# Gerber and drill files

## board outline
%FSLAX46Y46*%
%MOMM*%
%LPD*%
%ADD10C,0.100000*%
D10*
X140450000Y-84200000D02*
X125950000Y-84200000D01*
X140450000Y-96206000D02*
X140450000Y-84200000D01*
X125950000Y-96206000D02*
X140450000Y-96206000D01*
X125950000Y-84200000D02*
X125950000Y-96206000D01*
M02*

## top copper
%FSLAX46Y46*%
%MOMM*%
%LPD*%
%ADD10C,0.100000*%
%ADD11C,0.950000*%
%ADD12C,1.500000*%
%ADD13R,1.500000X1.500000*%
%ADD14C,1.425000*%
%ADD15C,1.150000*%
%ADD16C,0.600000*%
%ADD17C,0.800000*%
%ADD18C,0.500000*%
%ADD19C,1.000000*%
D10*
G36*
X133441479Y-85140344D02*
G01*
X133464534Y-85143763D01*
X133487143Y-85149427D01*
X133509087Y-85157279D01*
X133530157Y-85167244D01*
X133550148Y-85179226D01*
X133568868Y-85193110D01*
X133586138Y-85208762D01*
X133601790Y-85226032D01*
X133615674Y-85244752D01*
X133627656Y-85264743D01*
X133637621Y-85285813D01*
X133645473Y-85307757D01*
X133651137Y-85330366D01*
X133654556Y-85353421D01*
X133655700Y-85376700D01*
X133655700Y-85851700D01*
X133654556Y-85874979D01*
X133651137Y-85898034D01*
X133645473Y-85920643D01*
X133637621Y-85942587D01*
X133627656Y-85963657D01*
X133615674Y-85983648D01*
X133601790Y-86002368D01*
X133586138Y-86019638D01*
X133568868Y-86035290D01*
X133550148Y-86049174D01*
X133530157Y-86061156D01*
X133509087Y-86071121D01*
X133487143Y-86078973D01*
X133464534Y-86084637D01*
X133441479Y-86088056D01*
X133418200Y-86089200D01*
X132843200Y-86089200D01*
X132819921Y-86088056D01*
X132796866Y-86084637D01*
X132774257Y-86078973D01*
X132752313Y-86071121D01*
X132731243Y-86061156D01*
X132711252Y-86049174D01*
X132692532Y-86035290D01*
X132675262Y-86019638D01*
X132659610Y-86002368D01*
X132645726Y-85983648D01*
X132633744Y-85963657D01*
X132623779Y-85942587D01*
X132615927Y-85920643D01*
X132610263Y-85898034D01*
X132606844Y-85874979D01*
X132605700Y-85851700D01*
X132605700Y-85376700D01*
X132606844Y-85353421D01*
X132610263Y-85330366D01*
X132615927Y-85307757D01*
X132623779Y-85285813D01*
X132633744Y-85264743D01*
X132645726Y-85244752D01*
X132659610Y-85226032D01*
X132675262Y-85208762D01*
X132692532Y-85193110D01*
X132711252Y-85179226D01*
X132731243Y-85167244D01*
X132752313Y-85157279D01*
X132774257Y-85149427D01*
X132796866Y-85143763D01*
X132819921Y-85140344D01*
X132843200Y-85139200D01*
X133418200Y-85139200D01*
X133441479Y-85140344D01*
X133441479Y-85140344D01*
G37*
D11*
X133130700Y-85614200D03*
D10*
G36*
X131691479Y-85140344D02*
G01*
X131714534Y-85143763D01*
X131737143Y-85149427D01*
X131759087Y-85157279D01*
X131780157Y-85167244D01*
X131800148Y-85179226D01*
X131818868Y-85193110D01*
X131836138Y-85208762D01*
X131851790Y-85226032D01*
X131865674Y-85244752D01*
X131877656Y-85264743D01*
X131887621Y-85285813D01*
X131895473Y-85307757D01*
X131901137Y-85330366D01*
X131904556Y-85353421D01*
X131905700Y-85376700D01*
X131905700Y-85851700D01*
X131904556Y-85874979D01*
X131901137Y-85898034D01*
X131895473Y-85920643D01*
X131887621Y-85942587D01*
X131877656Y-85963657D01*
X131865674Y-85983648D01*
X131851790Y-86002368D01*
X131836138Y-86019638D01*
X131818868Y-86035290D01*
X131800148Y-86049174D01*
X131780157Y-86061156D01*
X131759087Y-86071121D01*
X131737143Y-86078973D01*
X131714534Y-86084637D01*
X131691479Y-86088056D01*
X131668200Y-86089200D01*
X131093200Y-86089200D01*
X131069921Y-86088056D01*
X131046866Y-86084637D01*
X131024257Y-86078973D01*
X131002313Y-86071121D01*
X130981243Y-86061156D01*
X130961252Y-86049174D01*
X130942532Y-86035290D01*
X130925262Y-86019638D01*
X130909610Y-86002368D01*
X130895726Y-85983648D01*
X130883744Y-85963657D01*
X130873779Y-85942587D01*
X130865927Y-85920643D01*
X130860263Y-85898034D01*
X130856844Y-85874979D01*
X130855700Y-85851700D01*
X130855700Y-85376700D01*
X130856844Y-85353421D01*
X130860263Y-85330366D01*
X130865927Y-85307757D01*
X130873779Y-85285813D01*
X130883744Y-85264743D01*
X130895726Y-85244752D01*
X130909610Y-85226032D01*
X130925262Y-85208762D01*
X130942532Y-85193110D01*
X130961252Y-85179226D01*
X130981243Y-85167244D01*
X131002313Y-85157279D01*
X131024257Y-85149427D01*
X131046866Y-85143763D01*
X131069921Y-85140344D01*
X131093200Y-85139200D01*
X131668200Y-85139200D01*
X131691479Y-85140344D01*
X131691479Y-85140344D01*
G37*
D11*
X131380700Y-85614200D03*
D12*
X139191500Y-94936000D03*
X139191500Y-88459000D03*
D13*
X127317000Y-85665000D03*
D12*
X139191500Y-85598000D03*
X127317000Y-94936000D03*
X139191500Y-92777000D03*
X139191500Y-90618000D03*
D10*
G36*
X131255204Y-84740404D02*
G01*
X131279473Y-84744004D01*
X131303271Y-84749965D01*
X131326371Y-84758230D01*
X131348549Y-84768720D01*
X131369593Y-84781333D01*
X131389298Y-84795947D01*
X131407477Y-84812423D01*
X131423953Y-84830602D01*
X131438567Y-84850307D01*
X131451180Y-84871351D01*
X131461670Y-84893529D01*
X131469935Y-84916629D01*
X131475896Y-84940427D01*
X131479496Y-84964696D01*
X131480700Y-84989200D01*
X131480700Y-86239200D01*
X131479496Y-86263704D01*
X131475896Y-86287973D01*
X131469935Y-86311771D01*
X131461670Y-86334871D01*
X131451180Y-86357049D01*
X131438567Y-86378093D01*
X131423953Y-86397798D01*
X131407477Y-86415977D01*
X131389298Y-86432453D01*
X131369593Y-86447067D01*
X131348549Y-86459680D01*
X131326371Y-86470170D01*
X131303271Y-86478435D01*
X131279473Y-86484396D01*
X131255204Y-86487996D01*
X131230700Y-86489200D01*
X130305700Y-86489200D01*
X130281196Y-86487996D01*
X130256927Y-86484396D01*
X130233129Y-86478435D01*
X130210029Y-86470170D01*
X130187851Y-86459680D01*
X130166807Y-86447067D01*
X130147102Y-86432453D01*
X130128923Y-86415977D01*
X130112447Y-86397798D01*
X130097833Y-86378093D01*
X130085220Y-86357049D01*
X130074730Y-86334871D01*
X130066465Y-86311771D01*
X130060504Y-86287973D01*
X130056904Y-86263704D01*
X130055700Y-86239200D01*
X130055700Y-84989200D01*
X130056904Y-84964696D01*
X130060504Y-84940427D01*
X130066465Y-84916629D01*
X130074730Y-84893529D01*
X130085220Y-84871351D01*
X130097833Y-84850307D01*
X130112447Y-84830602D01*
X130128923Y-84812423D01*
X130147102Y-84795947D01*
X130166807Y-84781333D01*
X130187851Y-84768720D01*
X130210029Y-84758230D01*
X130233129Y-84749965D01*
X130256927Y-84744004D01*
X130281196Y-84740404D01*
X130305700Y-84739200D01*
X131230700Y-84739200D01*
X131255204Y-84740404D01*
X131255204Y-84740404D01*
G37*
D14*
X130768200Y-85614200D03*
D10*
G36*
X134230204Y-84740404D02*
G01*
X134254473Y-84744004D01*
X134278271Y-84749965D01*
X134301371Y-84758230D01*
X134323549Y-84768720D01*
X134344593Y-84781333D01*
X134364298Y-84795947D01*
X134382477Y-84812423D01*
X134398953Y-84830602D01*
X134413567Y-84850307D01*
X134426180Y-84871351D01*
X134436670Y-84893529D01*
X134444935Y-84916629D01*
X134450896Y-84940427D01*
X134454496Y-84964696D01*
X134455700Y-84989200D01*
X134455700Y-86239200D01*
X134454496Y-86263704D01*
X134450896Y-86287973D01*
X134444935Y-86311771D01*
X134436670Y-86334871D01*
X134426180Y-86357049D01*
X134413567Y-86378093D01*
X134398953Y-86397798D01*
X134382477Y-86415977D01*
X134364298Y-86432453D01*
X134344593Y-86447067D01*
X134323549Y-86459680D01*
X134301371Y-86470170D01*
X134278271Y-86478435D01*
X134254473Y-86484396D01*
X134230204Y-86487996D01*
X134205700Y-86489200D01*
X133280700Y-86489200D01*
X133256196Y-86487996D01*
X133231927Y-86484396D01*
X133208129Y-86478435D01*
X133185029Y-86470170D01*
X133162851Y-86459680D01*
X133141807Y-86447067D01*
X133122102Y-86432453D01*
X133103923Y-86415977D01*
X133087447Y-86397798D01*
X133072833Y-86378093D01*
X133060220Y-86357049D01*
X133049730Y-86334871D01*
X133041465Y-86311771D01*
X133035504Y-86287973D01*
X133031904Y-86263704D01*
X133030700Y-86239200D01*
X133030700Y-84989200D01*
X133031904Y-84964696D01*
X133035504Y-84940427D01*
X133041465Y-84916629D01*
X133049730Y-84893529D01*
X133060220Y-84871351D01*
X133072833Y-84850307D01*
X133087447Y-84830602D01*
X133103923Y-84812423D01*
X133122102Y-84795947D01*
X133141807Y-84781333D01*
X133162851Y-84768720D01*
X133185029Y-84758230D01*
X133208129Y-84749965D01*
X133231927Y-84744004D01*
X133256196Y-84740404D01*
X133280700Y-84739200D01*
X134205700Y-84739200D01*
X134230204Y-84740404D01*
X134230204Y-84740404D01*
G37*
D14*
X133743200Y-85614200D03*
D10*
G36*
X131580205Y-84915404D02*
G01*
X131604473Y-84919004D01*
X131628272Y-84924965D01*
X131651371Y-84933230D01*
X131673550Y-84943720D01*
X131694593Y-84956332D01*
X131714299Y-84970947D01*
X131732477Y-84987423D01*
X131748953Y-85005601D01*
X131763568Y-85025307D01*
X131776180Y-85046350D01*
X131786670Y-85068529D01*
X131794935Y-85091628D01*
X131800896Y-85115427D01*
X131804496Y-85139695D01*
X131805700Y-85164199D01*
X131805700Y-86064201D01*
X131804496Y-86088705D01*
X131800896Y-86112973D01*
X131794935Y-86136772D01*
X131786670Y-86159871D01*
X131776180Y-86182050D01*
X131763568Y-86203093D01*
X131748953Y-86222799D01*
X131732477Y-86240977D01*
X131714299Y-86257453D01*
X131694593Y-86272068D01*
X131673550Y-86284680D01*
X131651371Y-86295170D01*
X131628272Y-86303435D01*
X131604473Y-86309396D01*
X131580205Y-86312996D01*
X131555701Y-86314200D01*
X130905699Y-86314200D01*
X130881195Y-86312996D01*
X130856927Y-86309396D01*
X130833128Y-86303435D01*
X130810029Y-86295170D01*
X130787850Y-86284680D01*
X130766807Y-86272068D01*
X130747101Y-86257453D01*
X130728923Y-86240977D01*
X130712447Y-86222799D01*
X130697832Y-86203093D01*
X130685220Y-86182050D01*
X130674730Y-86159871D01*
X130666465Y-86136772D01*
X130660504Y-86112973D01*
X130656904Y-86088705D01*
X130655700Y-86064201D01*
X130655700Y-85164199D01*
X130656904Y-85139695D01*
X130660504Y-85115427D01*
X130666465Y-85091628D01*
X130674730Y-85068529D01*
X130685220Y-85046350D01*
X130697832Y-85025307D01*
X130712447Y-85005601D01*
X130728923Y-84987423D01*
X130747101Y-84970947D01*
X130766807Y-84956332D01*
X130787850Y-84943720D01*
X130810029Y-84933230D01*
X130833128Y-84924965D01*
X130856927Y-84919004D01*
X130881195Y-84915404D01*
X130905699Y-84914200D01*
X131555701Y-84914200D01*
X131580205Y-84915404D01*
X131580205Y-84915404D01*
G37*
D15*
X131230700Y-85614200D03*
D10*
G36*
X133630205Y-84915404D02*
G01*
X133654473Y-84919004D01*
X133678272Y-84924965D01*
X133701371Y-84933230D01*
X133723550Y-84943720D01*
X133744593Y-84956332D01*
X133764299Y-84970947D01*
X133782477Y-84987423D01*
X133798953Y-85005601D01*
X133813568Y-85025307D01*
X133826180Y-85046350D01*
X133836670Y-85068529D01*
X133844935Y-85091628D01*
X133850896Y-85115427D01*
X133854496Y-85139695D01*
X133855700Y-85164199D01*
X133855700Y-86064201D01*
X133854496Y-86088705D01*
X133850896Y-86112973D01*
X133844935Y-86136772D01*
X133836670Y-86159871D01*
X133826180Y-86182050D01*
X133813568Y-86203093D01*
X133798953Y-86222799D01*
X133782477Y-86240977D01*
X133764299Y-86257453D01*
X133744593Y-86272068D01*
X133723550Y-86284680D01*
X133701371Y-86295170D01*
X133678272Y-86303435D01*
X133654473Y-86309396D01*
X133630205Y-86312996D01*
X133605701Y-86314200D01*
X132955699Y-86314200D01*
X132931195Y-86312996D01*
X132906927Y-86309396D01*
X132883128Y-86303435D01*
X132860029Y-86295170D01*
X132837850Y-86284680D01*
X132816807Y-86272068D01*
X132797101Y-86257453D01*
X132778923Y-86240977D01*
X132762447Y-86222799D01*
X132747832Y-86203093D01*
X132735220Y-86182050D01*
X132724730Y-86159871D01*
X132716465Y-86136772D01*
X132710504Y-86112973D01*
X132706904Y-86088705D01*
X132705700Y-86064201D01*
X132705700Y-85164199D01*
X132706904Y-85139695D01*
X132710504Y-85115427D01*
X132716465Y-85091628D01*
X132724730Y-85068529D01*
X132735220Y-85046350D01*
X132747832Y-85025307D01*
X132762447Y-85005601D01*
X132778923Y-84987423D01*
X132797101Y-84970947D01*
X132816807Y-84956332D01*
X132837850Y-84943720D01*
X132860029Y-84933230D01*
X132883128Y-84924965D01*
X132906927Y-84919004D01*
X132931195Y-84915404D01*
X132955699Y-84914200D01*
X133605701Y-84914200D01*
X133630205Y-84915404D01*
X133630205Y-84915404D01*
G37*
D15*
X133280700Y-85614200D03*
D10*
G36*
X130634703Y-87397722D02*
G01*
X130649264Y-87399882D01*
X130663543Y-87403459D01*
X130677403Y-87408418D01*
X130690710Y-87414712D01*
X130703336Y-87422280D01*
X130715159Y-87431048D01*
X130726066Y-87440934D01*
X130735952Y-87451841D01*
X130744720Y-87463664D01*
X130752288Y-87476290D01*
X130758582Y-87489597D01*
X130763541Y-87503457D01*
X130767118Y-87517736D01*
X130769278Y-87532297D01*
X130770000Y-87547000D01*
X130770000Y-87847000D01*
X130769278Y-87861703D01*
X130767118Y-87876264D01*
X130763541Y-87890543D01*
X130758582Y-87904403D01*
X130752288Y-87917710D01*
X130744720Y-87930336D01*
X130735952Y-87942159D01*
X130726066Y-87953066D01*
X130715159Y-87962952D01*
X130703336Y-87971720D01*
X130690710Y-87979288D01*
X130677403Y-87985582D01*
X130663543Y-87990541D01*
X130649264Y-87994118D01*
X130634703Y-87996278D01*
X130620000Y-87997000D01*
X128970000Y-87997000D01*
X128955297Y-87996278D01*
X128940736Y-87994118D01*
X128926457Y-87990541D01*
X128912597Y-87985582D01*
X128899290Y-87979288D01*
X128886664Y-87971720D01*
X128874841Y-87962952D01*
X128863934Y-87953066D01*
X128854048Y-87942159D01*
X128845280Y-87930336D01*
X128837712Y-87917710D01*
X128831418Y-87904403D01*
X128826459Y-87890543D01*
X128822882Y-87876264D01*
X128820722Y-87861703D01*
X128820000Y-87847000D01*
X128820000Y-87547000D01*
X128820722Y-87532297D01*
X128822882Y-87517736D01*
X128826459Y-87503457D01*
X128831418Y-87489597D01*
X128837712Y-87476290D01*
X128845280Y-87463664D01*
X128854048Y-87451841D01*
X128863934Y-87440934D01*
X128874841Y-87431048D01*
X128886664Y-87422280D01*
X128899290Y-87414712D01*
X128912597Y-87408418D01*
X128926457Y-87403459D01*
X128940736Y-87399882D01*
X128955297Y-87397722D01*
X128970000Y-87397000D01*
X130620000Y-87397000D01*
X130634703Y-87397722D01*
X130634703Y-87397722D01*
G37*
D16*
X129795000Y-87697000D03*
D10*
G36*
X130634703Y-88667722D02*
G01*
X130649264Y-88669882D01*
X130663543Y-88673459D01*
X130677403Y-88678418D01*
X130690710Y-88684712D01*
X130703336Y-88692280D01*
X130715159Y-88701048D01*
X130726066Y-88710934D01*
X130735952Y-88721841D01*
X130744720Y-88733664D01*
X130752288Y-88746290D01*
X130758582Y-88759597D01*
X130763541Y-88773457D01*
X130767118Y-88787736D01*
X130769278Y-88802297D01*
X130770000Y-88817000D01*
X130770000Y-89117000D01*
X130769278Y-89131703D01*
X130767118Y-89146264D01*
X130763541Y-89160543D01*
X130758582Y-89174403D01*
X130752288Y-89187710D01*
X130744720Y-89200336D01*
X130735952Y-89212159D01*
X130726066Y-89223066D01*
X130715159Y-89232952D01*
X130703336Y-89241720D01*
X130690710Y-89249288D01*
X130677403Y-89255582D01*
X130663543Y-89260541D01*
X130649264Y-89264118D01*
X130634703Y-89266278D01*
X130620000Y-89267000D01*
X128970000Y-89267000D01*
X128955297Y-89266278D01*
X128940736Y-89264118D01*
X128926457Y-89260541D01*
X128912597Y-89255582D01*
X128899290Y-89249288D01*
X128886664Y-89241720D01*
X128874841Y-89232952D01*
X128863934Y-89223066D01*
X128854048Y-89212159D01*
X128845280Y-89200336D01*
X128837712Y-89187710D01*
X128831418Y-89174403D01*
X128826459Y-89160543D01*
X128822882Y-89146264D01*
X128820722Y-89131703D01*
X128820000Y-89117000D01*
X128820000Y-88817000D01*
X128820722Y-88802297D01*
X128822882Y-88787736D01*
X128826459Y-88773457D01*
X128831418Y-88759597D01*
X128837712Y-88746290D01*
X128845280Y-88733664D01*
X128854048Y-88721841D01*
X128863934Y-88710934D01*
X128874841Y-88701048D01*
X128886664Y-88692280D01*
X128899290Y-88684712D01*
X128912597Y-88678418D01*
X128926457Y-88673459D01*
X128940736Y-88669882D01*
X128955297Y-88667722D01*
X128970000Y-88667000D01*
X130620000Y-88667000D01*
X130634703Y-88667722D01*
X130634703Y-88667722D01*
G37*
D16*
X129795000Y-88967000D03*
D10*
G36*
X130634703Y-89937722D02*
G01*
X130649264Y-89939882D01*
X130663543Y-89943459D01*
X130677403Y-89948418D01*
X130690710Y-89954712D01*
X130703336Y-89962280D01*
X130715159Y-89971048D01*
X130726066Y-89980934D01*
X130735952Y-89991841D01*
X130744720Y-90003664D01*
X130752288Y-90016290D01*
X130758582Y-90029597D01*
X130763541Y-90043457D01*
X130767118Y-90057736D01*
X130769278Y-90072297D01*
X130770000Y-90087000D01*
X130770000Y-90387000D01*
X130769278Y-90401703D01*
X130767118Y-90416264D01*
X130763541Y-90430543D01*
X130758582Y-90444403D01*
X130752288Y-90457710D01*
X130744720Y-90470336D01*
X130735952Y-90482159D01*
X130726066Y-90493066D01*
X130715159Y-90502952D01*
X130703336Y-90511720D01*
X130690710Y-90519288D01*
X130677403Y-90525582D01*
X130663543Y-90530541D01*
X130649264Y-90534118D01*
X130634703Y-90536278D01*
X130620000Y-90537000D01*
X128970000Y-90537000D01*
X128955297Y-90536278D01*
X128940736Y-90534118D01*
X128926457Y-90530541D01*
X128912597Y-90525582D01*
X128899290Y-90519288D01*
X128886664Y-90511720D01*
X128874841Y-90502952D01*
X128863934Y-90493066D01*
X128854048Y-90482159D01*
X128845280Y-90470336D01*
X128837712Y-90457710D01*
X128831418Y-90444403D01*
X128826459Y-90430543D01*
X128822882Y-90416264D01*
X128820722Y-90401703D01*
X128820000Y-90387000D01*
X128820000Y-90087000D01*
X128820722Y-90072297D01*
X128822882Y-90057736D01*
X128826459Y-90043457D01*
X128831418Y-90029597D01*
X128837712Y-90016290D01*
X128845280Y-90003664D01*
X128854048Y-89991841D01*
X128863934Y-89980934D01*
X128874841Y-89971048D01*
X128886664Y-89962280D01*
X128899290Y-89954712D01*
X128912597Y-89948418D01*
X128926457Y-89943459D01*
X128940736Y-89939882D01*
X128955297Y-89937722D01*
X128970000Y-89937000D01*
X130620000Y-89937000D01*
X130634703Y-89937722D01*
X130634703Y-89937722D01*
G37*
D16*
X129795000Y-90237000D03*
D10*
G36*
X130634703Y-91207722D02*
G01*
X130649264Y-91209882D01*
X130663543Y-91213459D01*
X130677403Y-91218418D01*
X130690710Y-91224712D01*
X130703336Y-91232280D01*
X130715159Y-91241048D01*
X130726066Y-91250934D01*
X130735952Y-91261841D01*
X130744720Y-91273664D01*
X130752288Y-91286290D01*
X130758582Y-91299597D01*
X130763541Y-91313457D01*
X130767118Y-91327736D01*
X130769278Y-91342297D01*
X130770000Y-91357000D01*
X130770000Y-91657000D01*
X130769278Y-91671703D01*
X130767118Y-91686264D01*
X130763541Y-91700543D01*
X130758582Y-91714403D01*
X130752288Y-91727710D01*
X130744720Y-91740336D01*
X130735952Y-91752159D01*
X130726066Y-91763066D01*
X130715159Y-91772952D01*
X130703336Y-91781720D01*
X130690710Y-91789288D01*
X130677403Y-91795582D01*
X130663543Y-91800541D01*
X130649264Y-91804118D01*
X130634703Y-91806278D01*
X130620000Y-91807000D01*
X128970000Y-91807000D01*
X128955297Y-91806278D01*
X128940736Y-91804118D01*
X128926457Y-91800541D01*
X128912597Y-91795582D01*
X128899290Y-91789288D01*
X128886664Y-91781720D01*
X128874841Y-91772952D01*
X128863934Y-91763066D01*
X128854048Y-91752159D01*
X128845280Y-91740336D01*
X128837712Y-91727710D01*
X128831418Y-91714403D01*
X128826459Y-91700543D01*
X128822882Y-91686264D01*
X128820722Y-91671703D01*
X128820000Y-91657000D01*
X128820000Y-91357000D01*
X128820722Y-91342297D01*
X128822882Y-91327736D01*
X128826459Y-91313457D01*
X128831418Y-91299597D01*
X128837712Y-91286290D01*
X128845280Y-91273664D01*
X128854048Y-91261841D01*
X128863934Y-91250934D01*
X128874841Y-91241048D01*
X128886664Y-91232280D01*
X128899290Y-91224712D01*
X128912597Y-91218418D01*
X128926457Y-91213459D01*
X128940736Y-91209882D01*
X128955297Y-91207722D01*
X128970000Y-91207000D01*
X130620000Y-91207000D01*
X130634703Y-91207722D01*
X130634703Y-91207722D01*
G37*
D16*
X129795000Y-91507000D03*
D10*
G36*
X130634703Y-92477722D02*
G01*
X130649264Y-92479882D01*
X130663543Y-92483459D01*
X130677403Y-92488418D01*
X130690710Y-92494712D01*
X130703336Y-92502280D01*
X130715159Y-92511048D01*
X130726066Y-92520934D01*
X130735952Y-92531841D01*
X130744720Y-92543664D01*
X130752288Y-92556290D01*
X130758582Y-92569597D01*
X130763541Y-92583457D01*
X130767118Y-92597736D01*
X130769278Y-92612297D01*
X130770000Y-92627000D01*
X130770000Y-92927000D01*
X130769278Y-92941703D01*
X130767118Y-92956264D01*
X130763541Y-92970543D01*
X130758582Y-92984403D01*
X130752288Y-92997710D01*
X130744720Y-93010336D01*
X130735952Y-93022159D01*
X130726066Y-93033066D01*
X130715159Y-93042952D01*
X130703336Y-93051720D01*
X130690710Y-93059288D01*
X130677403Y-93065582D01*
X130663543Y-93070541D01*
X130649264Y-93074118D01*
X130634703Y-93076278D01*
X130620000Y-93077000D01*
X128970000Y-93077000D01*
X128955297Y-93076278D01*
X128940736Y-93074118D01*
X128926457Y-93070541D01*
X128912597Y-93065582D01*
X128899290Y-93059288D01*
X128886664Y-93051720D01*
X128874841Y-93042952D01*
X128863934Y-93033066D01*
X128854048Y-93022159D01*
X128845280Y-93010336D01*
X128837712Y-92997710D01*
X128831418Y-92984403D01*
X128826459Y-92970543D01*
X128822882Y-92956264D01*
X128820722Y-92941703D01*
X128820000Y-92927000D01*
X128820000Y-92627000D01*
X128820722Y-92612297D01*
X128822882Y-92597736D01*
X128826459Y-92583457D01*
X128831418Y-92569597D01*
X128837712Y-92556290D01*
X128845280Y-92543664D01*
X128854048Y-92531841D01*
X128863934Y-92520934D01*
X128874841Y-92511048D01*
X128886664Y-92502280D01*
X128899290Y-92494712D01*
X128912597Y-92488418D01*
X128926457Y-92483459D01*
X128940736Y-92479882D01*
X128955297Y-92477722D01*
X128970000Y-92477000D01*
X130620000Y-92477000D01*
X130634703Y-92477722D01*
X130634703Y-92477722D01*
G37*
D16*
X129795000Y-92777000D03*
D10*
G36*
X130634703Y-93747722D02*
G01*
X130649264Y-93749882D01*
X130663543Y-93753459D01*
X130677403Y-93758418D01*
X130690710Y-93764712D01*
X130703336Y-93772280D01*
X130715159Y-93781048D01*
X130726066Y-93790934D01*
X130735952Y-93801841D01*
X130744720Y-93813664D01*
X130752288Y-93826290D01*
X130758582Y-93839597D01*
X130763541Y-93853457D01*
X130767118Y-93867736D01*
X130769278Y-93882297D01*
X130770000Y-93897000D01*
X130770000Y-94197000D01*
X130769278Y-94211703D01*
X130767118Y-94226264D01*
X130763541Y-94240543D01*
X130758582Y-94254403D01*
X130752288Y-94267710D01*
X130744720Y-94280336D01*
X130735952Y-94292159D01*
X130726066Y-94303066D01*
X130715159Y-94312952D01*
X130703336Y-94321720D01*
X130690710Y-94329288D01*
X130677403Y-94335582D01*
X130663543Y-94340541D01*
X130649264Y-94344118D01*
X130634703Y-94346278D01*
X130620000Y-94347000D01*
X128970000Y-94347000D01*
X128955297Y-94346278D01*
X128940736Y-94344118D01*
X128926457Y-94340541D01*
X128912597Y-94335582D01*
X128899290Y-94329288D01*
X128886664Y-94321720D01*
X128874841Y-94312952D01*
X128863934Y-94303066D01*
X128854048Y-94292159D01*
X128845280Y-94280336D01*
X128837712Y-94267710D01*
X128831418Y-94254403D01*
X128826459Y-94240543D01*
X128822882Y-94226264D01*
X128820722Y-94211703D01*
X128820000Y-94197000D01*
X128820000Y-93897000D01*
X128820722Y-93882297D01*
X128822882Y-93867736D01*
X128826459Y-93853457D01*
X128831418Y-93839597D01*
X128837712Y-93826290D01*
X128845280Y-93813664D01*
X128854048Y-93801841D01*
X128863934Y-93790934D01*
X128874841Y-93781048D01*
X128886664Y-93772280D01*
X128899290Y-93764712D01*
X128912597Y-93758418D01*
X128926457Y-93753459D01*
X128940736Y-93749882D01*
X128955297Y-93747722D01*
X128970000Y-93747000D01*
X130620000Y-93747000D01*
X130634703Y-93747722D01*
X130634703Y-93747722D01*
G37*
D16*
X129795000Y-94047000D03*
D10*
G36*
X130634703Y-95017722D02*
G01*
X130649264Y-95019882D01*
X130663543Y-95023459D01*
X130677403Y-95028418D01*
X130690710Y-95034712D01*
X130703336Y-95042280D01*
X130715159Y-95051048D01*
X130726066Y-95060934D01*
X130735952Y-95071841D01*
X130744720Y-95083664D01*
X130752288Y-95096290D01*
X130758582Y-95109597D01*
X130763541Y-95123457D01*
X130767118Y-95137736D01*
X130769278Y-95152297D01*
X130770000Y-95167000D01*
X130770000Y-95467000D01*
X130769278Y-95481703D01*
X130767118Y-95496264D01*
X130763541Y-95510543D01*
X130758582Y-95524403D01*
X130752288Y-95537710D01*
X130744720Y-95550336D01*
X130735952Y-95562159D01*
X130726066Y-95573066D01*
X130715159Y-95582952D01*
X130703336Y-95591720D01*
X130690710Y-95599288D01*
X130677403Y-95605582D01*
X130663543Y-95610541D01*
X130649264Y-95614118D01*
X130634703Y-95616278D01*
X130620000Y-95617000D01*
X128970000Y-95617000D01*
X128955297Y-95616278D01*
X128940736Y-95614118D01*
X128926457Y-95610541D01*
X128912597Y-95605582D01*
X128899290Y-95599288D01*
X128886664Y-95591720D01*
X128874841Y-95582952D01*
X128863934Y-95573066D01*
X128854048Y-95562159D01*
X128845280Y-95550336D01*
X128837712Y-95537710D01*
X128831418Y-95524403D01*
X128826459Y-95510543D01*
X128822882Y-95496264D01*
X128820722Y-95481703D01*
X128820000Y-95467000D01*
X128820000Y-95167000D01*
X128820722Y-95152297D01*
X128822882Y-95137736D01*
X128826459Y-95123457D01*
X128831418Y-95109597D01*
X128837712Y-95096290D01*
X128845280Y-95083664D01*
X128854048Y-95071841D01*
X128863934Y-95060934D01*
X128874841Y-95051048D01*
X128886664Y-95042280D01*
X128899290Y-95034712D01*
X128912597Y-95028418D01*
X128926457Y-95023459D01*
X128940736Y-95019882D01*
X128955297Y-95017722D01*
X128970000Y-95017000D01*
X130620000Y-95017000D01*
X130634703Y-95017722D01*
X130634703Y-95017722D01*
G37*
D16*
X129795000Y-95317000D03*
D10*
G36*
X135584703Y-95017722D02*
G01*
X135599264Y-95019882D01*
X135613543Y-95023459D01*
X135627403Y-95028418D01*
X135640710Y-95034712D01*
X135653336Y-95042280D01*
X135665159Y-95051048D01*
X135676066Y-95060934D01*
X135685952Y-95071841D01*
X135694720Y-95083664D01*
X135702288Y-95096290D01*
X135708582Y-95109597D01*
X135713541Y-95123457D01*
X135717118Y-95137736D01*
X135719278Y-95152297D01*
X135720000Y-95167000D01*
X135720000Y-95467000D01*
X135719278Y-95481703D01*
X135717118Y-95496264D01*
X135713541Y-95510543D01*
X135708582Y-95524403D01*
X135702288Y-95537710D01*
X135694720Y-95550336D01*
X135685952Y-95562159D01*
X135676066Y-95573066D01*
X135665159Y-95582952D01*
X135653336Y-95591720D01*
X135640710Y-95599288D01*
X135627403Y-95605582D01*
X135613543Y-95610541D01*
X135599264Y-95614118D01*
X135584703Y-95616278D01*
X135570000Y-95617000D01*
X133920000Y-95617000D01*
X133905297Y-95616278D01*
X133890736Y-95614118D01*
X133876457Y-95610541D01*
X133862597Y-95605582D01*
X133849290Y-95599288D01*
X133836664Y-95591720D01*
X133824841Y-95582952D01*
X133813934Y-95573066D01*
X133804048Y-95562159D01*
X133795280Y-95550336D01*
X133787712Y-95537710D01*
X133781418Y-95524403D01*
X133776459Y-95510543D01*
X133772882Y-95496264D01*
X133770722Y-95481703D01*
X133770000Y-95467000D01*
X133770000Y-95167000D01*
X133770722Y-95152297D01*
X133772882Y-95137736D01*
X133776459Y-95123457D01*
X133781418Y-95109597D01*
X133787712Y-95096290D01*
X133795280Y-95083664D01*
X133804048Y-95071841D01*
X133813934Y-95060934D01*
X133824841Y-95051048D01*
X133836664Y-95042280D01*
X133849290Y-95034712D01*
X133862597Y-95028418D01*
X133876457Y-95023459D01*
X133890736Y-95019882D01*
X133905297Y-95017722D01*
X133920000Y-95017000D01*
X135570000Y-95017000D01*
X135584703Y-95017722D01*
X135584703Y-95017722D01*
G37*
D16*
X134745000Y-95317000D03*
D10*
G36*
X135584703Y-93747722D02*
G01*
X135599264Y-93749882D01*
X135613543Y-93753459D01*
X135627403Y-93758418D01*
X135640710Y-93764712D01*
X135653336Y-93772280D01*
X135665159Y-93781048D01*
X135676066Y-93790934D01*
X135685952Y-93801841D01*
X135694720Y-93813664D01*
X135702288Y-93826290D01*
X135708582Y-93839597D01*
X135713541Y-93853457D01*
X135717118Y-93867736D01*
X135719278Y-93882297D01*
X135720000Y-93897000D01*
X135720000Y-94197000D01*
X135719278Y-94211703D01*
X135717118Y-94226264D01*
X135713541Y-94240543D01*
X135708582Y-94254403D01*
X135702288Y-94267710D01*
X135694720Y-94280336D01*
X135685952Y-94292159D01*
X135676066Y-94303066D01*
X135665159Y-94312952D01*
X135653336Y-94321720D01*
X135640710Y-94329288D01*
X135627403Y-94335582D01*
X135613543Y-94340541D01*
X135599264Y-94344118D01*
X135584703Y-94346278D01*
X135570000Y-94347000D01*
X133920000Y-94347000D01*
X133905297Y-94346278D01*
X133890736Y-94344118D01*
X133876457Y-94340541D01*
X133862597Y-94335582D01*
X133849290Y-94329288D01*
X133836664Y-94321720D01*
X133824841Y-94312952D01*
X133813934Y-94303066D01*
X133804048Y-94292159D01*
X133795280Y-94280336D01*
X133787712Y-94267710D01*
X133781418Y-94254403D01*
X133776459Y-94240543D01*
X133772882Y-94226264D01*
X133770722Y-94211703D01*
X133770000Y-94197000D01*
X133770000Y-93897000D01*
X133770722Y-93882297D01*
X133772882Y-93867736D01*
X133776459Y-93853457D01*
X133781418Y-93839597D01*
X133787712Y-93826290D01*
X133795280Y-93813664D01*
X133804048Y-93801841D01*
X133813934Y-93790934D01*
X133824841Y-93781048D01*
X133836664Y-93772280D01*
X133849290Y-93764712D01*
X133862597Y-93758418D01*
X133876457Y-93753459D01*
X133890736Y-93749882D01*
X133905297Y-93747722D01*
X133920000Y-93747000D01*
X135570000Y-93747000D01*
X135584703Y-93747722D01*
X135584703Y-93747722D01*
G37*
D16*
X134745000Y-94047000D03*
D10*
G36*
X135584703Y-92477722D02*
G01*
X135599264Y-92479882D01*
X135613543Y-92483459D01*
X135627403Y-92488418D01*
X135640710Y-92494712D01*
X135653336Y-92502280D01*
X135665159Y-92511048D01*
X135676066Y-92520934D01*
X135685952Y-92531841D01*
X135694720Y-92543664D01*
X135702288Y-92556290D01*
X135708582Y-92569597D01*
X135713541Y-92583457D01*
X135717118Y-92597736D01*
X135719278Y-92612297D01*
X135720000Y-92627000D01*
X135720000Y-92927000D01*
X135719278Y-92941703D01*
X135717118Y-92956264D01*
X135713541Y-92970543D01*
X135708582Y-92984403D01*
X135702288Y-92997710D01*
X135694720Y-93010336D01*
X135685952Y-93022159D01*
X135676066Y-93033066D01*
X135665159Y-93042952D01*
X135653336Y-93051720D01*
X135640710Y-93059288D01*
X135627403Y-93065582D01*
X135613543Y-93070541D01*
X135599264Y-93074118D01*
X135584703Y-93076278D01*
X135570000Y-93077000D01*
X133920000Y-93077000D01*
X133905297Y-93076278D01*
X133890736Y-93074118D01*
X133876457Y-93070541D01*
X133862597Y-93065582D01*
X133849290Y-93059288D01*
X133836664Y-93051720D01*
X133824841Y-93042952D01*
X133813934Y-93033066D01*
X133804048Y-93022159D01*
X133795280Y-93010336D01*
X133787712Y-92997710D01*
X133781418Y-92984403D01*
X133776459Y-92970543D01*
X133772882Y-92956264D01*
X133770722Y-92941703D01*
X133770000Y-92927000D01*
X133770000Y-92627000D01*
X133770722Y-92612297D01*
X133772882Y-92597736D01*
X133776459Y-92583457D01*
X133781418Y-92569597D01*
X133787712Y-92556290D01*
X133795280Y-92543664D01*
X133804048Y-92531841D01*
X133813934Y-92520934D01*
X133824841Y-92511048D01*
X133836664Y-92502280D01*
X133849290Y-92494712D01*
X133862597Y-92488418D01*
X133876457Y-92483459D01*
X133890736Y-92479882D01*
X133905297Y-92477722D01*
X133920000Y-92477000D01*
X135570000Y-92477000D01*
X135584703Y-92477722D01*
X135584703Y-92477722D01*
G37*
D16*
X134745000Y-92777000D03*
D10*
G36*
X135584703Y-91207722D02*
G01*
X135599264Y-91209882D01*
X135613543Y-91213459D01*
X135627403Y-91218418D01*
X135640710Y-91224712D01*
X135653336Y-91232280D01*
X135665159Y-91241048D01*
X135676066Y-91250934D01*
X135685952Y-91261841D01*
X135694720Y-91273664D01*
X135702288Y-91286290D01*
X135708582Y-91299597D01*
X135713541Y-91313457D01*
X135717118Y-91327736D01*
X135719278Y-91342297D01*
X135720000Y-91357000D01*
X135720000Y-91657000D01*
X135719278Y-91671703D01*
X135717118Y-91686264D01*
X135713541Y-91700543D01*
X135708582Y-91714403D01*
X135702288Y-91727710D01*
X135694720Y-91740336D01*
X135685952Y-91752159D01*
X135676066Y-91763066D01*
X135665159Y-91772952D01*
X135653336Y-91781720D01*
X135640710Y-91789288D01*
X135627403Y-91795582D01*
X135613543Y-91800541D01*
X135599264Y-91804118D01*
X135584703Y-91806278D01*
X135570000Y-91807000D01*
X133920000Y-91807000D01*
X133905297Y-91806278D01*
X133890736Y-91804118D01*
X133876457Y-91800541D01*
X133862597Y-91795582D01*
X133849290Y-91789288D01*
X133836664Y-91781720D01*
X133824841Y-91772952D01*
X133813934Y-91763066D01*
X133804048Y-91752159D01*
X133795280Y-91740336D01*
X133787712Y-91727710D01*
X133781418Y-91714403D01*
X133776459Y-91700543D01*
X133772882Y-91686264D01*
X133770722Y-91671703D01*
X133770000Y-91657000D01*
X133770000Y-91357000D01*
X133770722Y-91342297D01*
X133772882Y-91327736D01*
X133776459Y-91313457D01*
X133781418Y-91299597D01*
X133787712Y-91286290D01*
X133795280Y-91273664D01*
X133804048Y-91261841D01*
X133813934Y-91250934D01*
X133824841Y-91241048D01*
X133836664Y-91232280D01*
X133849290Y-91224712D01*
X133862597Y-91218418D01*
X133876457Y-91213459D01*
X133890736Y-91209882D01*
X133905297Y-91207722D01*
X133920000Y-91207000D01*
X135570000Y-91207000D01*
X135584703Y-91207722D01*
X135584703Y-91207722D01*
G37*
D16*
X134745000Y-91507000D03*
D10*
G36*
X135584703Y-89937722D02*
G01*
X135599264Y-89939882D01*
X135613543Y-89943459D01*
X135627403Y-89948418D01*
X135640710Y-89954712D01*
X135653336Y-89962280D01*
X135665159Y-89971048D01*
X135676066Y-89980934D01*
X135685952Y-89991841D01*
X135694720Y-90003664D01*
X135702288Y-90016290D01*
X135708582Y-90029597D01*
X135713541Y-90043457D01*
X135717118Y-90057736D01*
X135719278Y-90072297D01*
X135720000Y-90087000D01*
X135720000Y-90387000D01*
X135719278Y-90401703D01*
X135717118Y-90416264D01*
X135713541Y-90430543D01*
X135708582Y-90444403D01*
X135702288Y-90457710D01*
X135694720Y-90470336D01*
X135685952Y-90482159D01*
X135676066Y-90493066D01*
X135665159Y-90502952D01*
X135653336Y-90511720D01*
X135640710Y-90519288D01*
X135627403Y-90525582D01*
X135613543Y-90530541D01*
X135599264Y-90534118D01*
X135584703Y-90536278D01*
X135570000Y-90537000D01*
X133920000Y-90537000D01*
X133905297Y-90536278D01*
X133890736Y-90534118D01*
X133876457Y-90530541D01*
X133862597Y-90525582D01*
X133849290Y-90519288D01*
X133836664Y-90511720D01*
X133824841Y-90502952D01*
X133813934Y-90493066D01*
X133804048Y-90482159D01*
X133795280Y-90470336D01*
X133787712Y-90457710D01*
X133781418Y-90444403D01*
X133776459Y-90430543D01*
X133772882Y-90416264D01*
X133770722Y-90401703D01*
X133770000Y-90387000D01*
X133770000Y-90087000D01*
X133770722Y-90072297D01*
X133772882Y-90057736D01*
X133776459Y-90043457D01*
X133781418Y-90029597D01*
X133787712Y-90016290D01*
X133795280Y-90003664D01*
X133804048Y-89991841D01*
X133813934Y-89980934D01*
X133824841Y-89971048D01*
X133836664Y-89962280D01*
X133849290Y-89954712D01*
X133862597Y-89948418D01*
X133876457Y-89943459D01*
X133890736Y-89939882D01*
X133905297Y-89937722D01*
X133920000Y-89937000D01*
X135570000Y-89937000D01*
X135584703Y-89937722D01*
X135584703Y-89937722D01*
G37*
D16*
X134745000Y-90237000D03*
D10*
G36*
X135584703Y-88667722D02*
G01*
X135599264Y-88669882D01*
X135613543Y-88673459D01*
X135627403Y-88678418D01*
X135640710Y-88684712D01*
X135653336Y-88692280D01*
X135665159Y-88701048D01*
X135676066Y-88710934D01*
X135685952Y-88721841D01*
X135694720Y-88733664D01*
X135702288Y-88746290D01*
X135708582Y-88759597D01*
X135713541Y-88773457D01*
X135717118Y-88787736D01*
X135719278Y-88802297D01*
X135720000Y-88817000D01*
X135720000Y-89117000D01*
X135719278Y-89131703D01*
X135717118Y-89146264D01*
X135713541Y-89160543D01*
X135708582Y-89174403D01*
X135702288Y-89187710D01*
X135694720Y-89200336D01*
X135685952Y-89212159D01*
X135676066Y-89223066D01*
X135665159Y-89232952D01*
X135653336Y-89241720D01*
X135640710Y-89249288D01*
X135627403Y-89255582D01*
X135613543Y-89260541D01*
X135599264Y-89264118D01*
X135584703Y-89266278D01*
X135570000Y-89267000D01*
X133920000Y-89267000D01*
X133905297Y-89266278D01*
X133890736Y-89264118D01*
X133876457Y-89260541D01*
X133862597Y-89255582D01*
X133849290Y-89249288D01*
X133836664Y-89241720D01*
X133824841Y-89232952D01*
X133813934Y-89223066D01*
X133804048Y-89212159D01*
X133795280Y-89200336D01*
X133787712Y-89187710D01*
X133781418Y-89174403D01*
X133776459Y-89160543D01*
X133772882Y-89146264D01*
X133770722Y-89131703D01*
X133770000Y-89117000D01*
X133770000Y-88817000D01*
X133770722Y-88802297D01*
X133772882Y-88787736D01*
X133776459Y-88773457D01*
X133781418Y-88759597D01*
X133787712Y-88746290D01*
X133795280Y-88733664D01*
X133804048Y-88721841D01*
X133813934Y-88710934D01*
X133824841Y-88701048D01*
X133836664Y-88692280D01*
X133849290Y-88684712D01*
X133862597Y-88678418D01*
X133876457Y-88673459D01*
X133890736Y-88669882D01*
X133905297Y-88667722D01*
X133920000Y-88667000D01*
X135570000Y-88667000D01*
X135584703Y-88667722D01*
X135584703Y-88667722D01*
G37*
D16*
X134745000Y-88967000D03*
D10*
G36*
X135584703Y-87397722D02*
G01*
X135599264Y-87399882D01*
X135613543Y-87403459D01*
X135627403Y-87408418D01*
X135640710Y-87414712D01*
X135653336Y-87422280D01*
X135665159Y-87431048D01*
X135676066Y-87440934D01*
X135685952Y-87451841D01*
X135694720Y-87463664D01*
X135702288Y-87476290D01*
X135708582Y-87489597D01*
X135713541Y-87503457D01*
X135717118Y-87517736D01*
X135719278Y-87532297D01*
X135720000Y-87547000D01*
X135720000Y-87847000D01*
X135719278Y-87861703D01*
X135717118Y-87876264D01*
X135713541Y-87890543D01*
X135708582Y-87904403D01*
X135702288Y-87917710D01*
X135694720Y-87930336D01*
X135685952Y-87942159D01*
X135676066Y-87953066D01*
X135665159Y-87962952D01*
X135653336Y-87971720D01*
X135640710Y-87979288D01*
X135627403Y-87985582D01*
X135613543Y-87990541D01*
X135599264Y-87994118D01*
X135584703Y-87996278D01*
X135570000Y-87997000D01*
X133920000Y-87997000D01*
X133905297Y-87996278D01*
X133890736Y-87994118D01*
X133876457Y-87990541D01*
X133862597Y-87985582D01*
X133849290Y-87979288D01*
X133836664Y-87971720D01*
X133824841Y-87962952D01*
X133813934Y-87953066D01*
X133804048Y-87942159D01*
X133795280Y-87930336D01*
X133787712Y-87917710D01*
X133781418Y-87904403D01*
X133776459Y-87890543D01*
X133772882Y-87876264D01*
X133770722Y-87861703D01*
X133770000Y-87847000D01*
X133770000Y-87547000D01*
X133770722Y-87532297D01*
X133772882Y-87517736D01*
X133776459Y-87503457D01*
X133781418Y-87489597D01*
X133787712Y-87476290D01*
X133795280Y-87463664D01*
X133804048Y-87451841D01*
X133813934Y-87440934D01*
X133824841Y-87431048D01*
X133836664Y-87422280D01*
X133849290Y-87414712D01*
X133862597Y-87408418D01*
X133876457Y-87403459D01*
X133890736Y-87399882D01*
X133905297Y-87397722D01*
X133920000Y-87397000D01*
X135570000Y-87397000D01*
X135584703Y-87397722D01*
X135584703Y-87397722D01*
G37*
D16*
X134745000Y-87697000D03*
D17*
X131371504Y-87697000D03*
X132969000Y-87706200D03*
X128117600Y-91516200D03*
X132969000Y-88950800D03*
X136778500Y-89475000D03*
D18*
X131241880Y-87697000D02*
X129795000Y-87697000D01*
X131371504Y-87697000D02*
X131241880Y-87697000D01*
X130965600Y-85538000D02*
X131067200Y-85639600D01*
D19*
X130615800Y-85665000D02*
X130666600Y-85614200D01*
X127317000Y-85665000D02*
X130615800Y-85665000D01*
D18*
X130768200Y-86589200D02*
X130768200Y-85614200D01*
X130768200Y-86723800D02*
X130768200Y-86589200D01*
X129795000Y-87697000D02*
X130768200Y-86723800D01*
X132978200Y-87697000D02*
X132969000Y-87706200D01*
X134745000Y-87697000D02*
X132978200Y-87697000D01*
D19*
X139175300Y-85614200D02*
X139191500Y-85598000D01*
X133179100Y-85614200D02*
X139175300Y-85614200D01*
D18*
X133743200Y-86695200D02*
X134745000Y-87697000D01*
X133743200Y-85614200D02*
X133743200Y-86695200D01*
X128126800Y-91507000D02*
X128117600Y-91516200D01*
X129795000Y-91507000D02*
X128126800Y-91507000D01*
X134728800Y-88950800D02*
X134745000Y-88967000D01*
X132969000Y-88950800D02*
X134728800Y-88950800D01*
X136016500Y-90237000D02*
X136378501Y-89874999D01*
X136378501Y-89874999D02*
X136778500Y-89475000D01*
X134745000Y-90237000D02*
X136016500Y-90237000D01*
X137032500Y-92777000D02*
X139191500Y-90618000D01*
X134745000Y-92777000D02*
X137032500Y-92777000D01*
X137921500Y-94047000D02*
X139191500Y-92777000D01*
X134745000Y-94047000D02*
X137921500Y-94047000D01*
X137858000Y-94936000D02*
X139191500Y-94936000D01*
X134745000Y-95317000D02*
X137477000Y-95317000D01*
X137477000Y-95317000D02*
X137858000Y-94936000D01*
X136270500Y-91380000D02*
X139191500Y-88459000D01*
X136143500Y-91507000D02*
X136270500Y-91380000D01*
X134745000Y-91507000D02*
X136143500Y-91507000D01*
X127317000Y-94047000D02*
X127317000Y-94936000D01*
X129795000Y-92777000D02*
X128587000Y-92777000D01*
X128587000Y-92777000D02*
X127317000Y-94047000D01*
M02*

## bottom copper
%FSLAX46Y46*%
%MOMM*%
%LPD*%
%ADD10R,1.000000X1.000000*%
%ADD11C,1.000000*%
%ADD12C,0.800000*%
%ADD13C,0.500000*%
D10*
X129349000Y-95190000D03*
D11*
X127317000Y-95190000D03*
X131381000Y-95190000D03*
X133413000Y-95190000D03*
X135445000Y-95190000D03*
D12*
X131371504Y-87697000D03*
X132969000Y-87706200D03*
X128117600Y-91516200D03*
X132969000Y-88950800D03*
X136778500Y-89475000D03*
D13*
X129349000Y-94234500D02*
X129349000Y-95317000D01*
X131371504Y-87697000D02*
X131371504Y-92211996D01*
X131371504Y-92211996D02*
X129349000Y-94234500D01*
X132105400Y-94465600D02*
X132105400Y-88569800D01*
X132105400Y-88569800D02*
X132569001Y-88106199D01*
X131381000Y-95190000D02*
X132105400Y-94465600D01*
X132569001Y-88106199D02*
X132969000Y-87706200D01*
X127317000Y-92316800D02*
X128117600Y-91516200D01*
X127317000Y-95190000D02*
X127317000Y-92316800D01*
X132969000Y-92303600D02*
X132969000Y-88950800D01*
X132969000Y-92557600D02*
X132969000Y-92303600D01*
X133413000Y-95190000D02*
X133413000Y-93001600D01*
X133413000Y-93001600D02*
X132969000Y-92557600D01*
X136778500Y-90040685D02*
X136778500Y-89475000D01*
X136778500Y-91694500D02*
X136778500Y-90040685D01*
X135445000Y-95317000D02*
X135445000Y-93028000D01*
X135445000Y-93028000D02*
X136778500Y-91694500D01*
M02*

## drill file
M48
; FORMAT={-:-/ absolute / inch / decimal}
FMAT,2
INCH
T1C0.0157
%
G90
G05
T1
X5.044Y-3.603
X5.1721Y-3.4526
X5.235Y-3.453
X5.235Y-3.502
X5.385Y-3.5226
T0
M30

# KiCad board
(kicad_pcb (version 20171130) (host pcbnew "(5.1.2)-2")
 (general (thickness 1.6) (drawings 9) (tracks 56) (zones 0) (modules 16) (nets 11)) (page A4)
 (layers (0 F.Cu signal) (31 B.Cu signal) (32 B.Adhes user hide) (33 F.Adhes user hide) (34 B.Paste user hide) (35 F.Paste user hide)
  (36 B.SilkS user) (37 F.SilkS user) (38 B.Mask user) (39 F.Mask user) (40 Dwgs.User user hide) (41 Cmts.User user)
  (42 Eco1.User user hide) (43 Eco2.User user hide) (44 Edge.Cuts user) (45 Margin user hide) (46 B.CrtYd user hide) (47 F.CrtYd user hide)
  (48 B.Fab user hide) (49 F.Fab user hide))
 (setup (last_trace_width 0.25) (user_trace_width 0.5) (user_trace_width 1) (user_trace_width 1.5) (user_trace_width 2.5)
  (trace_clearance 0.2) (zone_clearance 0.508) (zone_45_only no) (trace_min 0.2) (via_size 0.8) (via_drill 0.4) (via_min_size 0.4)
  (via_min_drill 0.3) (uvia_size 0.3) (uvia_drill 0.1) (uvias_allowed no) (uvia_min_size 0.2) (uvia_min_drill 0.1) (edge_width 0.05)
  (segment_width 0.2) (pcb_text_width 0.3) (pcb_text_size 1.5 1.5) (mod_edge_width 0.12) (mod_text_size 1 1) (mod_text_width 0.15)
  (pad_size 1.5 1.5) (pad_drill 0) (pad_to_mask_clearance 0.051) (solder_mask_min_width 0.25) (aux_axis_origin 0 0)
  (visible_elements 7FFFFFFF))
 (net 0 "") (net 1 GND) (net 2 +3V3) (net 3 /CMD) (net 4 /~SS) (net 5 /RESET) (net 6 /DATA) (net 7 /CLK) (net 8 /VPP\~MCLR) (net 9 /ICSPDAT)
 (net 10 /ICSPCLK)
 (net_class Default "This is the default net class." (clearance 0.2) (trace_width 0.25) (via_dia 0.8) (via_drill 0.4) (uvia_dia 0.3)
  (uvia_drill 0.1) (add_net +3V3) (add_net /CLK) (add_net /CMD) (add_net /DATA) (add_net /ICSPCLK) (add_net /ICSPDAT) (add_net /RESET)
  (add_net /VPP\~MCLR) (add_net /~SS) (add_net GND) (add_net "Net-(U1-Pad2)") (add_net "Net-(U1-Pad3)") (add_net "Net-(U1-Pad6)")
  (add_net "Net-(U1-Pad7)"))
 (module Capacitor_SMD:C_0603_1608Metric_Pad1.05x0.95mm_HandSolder (layer F.Cu) (at 132.2557 85.6142)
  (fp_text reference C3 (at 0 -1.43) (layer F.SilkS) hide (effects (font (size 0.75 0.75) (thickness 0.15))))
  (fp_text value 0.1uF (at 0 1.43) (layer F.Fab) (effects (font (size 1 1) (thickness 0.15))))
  (pad 2 smd roundrect (at 0.875 0) (size 1.05 0.95) (layers F.Cu F.Paste F.Mask) (roundrect_rratio 0.25) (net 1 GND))
  (pad 1 smd roundrect (at -0.875 0) (size 1.05 0.95) (layers F.Cu F.Paste F.Mask) (roundrect_rratio 0.25) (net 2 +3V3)))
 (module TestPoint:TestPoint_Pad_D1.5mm (layer F.Cu) (at 139.1915 94.936)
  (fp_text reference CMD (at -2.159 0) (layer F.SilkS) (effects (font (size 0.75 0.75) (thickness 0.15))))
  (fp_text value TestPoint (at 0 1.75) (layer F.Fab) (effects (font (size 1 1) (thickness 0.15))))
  (pad 1 smd circle (at 0 0) (size 1.5 1.5) (layers F.Cu F.Mask) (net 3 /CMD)))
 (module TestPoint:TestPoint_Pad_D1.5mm (layer F.Cu) (at 139.1915 88.459)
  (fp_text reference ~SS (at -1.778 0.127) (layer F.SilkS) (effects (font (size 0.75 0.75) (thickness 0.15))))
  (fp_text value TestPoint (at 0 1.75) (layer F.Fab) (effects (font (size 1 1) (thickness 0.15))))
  (pad 1 smd circle (at 0 0) (size 1.5 1.5) (layers F.Cu F.Mask) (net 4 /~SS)))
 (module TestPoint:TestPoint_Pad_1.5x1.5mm (layer F.Cu) (at 127.317 85.665)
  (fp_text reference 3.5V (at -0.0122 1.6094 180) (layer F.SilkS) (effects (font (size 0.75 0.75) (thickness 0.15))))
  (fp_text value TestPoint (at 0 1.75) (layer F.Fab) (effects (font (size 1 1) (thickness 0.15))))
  (pad 1 smd rect (at 0 0) (size 1.5 1.5) (layers F.Cu F.Mask) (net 2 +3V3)))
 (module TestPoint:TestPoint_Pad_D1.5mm (layer F.Cu) (at 139.1915 85.598)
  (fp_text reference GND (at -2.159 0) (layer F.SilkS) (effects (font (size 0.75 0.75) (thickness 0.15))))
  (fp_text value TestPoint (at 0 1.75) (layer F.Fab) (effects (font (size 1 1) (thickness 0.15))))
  (pad 1 smd circle (at 0 0) (size 1.5 1.5) (layers F.Cu F.Mask) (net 1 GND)))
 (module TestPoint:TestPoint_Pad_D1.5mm (layer F.Cu) (at 127.317 94.936)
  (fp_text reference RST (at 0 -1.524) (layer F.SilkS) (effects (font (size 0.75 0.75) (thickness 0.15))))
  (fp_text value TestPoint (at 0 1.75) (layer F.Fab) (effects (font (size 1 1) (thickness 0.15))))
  (pad 1 smd circle (at 0 0) (size 1.5 1.5) (layers F.Cu F.Mask) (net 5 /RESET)))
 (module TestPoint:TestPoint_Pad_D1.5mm (layer F.Cu) (at 139.1915 92.777)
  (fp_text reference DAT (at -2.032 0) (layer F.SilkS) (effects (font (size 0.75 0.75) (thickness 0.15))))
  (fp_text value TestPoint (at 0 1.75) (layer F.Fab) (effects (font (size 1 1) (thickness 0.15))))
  (pad 1 smd circle (at 0 0) (size 1.5 1.5) (layers F.Cu F.Mask) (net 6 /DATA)))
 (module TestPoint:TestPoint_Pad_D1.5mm (layer F.Cu) (at 139.1915 90.618)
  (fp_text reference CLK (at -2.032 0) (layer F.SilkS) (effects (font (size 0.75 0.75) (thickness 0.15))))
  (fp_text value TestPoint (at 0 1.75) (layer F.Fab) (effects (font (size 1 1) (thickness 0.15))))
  (pad 1 smd circle (at 0 0) (size 1.5 1.5) (layers F.Cu F.Mask) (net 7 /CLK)))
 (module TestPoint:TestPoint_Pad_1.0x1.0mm (layer B.Cu) (at 129.349 95.19)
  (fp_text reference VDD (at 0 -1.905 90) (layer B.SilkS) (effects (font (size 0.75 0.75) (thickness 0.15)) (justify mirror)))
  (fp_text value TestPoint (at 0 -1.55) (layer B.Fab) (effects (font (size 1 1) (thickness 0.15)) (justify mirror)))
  (pad 1 smd rect (at 0 0) (size 1 1) (layers B.Cu B.Mask) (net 2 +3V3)))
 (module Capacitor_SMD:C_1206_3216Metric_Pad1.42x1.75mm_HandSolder (layer F.Cu) (at 132.2557 85.6142)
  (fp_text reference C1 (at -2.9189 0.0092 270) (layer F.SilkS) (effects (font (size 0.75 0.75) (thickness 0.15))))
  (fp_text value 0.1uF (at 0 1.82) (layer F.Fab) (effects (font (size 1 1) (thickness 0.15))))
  (pad 1 smd roundrect (at -1.4875 0) (size 1.425 1.75) (layers F.Cu F.Paste F.Mask) (roundrect_rratio 0.175439) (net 2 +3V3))
  (pad 2 smd roundrect (at 1.4875 0) (size 1.425 1.75) (layers F.Cu F.Paste F.Mask) (roundrect_rratio 0.175439) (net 1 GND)))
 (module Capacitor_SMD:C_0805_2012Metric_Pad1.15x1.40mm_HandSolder (layer F.Cu) (at 132.2557 85.6142)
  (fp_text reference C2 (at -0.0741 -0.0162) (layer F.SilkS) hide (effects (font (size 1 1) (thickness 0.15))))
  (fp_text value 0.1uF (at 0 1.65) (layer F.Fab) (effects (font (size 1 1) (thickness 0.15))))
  (pad 1 smd roundrect (at -1.025 0) (size 1.15 1.4) (layers F.Cu F.Paste F.Mask) (roundrect_rratio 0.217391) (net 2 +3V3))
  (pad 2 smd roundrect (at 1.025 0) (size 1.15 1.4) (layers F.Cu F.Paste F.Mask) (roundrect_rratio 0.217391) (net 1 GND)))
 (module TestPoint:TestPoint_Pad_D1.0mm (layer B.Cu) (at 127.317 95.19)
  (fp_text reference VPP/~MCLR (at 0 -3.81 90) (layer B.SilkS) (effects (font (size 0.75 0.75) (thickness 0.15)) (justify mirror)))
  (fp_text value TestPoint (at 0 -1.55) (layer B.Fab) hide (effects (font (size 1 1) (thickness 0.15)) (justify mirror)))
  (pad 1 smd circle (at 0 0) (size 1 1) (layers B.Cu B.Mask) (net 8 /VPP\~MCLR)))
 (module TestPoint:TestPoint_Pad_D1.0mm (layer B.Cu) (at 131.381 95.19)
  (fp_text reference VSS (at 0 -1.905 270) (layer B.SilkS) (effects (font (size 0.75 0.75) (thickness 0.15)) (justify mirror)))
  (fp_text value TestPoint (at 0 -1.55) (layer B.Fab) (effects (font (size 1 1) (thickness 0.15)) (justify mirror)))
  (pad 1 smd circle (at 0 0) (size 1 1) (layers B.Cu B.Mask) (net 1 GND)))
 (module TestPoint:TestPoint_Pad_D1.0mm (layer B.Cu) (at 133.413 95.19)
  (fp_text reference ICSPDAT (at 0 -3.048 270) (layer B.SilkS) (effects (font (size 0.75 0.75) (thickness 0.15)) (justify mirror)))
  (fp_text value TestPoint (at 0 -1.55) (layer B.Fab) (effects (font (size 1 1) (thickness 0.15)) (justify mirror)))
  (pad 1 smd circle (at 0 0) (size 1 1) (layers B.Cu B.Mask) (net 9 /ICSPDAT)))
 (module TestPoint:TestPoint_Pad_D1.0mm (layer B.Cu) (at 135.445 95.19)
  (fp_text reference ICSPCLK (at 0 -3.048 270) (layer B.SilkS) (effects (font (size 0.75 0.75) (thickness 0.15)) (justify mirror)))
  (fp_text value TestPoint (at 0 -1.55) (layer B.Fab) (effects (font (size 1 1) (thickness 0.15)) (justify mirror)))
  (pad 1 smd circle (at 0 0) (size 1 1) (layers B.Cu B.Mask) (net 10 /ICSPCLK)))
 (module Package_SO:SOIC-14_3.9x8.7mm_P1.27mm (layer F.Cu) (at 132.27 91.507)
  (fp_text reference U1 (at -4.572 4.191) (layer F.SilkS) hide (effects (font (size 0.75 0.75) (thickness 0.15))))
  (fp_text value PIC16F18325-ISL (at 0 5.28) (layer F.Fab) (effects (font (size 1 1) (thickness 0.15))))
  (pad 1 smd roundrect (at -2.475 -3.81) (size 1.95 0.6) (layers F.Cu F.Paste F.Mask) (roundrect_rratio 0.25) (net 2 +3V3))
  (pad 2 smd roundrect (at -2.475 -2.54) (size 1.95 0.6) (layers F.Cu F.Paste F.Mask) (roundrect_rratio 0.25))
  (pad 3 smd roundrect (at -2.475 -1.27) (size 1.95 0.6) (layers F.Cu F.Paste F.Mask) (roundrect_rratio 0.25))
  (pad 4 smd roundrect (at -2.475 0) (size 1.95 0.6) (layers F.Cu F.Paste F.Mask) (roundrect_rratio 0.25) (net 8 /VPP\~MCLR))
  (pad 5 smd roundrect (at -2.475 1.27) (size 1.95 0.6) (layers F.Cu F.Paste F.Mask) (roundrect_rratio 0.25) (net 5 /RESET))
  (pad 6 smd roundrect (at -2.475 2.54) (size 1.95 0.6) (layers F.Cu F.Paste F.Mask) (roundrect_rratio 0.25))
  (pad 7 smd roundrect (at -2.475 3.81) (size 1.95 0.6) (layers F.Cu F.Paste F.Mask) (roundrect_rratio 0.25))
  (pad 8 smd roundrect (at 2.475 3.81) (size 1.95 0.6) (layers F.Cu F.Paste F.Mask) (roundrect_rratio 0.25) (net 3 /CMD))
  (pad 9 smd roundrect (at 2.475 2.54) (size 1.95 0.6) (layers F.Cu F.Paste F.Mask) (roundrect_rratio 0.25) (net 6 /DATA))
  (pad 10 smd roundrect (at 2.475 1.27) (size 1.95 0.6) (layers F.Cu F.Paste F.Mask) (roundrect_rratio 0.25) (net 7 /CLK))
  (pad 11 smd roundrect (at 2.475 0) (size 1.95 0.6) (layers F.Cu F.Paste F.Mask) (roundrect_rratio 0.25) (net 4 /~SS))
  (pad 12 smd roundrect (at 2.475 -1.27) (size 1.95 0.6) (layers F.Cu F.Paste F.Mask) (roundrect_rratio 0.25) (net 10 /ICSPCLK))
  (pad 13 smd roundrect (at 2.475 -2.54) (size 1.95 0.6) (layers F.Cu F.Paste F.Mask) (roundrect_rratio 0.25) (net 9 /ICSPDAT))
  (pad 14 smd roundrect (at 2.475 -3.81) (size 1.95 0.6) (layers F.Cu F.Paste F.Mask) (roundrect_rratio 0.25) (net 1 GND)))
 (gr_line (start 140.45 84.2) (end 125.95 84.2) (layer Edge.Cuts) (width 0.1))
 (gr_line (start 140.45 96.206) (end 140.45 84.2) (layer Edge.Cuts) (width 0.1))
 (gr_line (start 125.95 96.206) (end 140.45 96.206) (layer Edge.Cuts) (width 0.1))
 (gr_line (start 125.95 84.2) (end 125.95 96.206) (layer Edge.Cuts) (width 0.1))
 (via (at 131.371504 87.697) (size 0.8) (drill 0.4) (layers F.Cu B.Cu) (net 2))
 (segment (start 131.24188 87.697) (end 129.795 87.697) (width 0.5) (layer F.Cu) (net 2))
 (segment (start 131.371504 87.697) (end 131.24188 87.697) (width 0.5) (layer F.Cu) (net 2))
 (segment (start 130.9656 85.538) (end 131.0672 85.6396) (width 0.5) (layer F.Cu) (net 2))
 (segment (start 129.349 94.2345) (end 129.349 95.317) (width 0.5) (layer B.Cu) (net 2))
 (segment (start 131.371504 87.697) (end 131.371504 92.211996) (width 0.5) (layer B.Cu) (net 2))
 (segment (start 131.371504 92.211996) (end 129.349 94.2345) (width 0.5) (layer B.Cu) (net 2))
 (segment (start 130.6158 85.665) (end 130.6666 85.6142) (width 1) (layer F.Cu) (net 2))
 (segment (start 127.317 85.665) (end 130.6158 85.665) (width 1) (layer F.Cu) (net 2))
 (segment (start 130.7682 86.5892) (end 130.7682 85.6142) (width 0.5) (layer F.Cu) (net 2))
 (segment (start 130.7682 86.7238) (end 130.7682 86.5892) (width 0.5) (layer F.Cu) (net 2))
 (segment (start 129.795 87.697) (end 130.7682 86.7238) (width 0.5) (layer F.Cu) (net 2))
 (segment (start 132.1054 94.4656) (end 132.1054 88.5698) (width 0.5) (layer B.Cu) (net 1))
 (segment (start 132.1054 88.5698) (end 132.569001 88.106199) (width 0.5) (layer B.Cu) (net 1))
 (segment (start 131.381 95.19) (end 132.1054 94.4656) (width 0.5) (layer B.Cu) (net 1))
 (segment (start 132.9782 87.697) (end 132.969 87.7062) (width 0.5) (layer F.Cu) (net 1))
 (segment (start 134.745 87.697) (end 132.9782 87.697) (width 0.5) (layer F.Cu) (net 1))
 (via (at 132.969 87.7062) (size 0.8) (drill 0.4) (layers F.Cu B.Cu) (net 1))
 (segment (start 132.569001 88.106199) (end 132.969 87.7062) (width 0.5) (layer B.Cu) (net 1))
 (segment (start 139.1753 85.6142) (end 139.1915 85.598) (width 1) (layer F.Cu) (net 1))
 (segment (start 133.1791 85.6142) (end 139.1753 85.6142) (width 1) (layer F.Cu) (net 1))
 (segment (start 133.7432 86.6952) (end 134.745 87.697) (width 0.5) (layer F.Cu) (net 1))
 (segment (start 133.7432 85.6142) (end 133.7432 86.6952) (width 0.5) (layer F.Cu) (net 1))
 (via (at 128.1176 91.5162) (size 0.8) (drill 0.4) (layers F.Cu B.Cu) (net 8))
 (segment (start 128.1268 91.507) (end 128.1176 91.5162) (width 0.5) (layer F.Cu) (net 8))
 (segment (start 129.795 91.507) (end 128.1268 91.507) (width 0.5) (layer F.Cu) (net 8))
 (segment (start 127.317 92.3168) (end 128.1176 91.5162) (width 0.5) (layer B.Cu) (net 8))
 (segment (start 127.317 95.19) (end 127.317 92.3168) (width 0.5) (layer B.Cu) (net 8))
 (via (at 132.969 88.9508) (size 0.8) (drill 0.4) (layers F.Cu B.Cu) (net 9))
 (segment (start 134.7288 88.9508) (end 134.745 88.967) (width 0.5) (layer F.Cu) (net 9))
 (segment (start 132.969 88.9508) (end 134.7288 88.9508) (width 0.5) (layer F.Cu) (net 9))
 (segment (start 132.969 92.3036) (end 132.969 88.9508) (width 0.5) (layer B.Cu) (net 9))
 (segment (start 132.969 92.5576) (end 132.969 92.3036) (width 0.5) (layer B.Cu) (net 9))
 (segment (start 133.413 95.19) (end 133.413 93.0016) (width 0.5) (layer B.Cu) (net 9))
 (segment (start 133.413 93.0016) (end 132.969 92.5576) (width 0.5) (layer B.Cu) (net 9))
 (segment (start 136.0165 90.237) (end 136.378501 89.874999) (width 0.5) (layer F.Cu) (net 10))
 (via (at 136.7785 89.475) (size 0.8) (drill 0.4) (layers F.Cu B.Cu) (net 10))
 (segment (start 136.378501 89.874999) (end 136.7785 89.475) (width 0.5) (layer F.Cu) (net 10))
 (segment (start 134.745 90.237) (end 136.0165 90.237) (width 0.5) (layer F.Cu) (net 10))
 (segment (start 136.7785 90.040685) (end 136.7785 89.475) (width 0.5) (layer B.Cu) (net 10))
 (segment (start 136.7785 91.6945) (end 136.7785 90.040685) (width 0.5) (layer B.Cu) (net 10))
 (segment (start 135.445 95.317) (end 135.445 93.028) (width 0.5) (layer B.Cu) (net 10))
 (segment (start 135.445 93.028) (end 136.7785 91.6945) (width 0.5) (layer B.Cu) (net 10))
 (segment (start 137.0325 92.777) (end 139.1915 90.618) (width 0.5) (layer F.Cu) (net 7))
 (segment (start 134.745 92.777) (end 137.0325 92.777) (width 0.5) (layer F.Cu) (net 7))
 (segment (start 137.9215 94.047) (end 139.1915 92.777) (width 0.5) (layer F.Cu) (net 6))
 (segment (start 134.745 94.047) (end 137.9215 94.047) (width 0.5) (layer F.Cu) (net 6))
 (segment (start 137.858 94.936) (end 139.1915 94.936) (width 0.5) (layer F.Cu) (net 3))
 (segment (start 134.745 95.317) (end 137.477 95.317) (width 0.5) (layer F.Cu) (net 3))
 (segment (start 137.477 95.317) (end 137.858 94.936) (width 0.5) (layer F.Cu) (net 3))
 (segment (start 136.2705 91.38) (end 139.1915 88.459) (width 0.5) (layer F.Cu) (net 4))
 (segment (start 136.1435 91.507) (end 136.2705 91.38) (width 0.5) (layer F.Cu) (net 4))
 (segment (start 134.745 91.507) (end 136.1435 91.507) (width 0.5) (layer F.Cu) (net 4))
 (segment (start 127.317 94.047) (end 127.317 94.936) (width 0.5) (layer F.Cu) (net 5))
 (segment (start 129.795 92.777) (end 128.587 92.777) (width 0.5) (layer F.Cu) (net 5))
 (segment (start 128.587 92.777) (end 127.317 94.047) (width 0.5) (layer F.Cu) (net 5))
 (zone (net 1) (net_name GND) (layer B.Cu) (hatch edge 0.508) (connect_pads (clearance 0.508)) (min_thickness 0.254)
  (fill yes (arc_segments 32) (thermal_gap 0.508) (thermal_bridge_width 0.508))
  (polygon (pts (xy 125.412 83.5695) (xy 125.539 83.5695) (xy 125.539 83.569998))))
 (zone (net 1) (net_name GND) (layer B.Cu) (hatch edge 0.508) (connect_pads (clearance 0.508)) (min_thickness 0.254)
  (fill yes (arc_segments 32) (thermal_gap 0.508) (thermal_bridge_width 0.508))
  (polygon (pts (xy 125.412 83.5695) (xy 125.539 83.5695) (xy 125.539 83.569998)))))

